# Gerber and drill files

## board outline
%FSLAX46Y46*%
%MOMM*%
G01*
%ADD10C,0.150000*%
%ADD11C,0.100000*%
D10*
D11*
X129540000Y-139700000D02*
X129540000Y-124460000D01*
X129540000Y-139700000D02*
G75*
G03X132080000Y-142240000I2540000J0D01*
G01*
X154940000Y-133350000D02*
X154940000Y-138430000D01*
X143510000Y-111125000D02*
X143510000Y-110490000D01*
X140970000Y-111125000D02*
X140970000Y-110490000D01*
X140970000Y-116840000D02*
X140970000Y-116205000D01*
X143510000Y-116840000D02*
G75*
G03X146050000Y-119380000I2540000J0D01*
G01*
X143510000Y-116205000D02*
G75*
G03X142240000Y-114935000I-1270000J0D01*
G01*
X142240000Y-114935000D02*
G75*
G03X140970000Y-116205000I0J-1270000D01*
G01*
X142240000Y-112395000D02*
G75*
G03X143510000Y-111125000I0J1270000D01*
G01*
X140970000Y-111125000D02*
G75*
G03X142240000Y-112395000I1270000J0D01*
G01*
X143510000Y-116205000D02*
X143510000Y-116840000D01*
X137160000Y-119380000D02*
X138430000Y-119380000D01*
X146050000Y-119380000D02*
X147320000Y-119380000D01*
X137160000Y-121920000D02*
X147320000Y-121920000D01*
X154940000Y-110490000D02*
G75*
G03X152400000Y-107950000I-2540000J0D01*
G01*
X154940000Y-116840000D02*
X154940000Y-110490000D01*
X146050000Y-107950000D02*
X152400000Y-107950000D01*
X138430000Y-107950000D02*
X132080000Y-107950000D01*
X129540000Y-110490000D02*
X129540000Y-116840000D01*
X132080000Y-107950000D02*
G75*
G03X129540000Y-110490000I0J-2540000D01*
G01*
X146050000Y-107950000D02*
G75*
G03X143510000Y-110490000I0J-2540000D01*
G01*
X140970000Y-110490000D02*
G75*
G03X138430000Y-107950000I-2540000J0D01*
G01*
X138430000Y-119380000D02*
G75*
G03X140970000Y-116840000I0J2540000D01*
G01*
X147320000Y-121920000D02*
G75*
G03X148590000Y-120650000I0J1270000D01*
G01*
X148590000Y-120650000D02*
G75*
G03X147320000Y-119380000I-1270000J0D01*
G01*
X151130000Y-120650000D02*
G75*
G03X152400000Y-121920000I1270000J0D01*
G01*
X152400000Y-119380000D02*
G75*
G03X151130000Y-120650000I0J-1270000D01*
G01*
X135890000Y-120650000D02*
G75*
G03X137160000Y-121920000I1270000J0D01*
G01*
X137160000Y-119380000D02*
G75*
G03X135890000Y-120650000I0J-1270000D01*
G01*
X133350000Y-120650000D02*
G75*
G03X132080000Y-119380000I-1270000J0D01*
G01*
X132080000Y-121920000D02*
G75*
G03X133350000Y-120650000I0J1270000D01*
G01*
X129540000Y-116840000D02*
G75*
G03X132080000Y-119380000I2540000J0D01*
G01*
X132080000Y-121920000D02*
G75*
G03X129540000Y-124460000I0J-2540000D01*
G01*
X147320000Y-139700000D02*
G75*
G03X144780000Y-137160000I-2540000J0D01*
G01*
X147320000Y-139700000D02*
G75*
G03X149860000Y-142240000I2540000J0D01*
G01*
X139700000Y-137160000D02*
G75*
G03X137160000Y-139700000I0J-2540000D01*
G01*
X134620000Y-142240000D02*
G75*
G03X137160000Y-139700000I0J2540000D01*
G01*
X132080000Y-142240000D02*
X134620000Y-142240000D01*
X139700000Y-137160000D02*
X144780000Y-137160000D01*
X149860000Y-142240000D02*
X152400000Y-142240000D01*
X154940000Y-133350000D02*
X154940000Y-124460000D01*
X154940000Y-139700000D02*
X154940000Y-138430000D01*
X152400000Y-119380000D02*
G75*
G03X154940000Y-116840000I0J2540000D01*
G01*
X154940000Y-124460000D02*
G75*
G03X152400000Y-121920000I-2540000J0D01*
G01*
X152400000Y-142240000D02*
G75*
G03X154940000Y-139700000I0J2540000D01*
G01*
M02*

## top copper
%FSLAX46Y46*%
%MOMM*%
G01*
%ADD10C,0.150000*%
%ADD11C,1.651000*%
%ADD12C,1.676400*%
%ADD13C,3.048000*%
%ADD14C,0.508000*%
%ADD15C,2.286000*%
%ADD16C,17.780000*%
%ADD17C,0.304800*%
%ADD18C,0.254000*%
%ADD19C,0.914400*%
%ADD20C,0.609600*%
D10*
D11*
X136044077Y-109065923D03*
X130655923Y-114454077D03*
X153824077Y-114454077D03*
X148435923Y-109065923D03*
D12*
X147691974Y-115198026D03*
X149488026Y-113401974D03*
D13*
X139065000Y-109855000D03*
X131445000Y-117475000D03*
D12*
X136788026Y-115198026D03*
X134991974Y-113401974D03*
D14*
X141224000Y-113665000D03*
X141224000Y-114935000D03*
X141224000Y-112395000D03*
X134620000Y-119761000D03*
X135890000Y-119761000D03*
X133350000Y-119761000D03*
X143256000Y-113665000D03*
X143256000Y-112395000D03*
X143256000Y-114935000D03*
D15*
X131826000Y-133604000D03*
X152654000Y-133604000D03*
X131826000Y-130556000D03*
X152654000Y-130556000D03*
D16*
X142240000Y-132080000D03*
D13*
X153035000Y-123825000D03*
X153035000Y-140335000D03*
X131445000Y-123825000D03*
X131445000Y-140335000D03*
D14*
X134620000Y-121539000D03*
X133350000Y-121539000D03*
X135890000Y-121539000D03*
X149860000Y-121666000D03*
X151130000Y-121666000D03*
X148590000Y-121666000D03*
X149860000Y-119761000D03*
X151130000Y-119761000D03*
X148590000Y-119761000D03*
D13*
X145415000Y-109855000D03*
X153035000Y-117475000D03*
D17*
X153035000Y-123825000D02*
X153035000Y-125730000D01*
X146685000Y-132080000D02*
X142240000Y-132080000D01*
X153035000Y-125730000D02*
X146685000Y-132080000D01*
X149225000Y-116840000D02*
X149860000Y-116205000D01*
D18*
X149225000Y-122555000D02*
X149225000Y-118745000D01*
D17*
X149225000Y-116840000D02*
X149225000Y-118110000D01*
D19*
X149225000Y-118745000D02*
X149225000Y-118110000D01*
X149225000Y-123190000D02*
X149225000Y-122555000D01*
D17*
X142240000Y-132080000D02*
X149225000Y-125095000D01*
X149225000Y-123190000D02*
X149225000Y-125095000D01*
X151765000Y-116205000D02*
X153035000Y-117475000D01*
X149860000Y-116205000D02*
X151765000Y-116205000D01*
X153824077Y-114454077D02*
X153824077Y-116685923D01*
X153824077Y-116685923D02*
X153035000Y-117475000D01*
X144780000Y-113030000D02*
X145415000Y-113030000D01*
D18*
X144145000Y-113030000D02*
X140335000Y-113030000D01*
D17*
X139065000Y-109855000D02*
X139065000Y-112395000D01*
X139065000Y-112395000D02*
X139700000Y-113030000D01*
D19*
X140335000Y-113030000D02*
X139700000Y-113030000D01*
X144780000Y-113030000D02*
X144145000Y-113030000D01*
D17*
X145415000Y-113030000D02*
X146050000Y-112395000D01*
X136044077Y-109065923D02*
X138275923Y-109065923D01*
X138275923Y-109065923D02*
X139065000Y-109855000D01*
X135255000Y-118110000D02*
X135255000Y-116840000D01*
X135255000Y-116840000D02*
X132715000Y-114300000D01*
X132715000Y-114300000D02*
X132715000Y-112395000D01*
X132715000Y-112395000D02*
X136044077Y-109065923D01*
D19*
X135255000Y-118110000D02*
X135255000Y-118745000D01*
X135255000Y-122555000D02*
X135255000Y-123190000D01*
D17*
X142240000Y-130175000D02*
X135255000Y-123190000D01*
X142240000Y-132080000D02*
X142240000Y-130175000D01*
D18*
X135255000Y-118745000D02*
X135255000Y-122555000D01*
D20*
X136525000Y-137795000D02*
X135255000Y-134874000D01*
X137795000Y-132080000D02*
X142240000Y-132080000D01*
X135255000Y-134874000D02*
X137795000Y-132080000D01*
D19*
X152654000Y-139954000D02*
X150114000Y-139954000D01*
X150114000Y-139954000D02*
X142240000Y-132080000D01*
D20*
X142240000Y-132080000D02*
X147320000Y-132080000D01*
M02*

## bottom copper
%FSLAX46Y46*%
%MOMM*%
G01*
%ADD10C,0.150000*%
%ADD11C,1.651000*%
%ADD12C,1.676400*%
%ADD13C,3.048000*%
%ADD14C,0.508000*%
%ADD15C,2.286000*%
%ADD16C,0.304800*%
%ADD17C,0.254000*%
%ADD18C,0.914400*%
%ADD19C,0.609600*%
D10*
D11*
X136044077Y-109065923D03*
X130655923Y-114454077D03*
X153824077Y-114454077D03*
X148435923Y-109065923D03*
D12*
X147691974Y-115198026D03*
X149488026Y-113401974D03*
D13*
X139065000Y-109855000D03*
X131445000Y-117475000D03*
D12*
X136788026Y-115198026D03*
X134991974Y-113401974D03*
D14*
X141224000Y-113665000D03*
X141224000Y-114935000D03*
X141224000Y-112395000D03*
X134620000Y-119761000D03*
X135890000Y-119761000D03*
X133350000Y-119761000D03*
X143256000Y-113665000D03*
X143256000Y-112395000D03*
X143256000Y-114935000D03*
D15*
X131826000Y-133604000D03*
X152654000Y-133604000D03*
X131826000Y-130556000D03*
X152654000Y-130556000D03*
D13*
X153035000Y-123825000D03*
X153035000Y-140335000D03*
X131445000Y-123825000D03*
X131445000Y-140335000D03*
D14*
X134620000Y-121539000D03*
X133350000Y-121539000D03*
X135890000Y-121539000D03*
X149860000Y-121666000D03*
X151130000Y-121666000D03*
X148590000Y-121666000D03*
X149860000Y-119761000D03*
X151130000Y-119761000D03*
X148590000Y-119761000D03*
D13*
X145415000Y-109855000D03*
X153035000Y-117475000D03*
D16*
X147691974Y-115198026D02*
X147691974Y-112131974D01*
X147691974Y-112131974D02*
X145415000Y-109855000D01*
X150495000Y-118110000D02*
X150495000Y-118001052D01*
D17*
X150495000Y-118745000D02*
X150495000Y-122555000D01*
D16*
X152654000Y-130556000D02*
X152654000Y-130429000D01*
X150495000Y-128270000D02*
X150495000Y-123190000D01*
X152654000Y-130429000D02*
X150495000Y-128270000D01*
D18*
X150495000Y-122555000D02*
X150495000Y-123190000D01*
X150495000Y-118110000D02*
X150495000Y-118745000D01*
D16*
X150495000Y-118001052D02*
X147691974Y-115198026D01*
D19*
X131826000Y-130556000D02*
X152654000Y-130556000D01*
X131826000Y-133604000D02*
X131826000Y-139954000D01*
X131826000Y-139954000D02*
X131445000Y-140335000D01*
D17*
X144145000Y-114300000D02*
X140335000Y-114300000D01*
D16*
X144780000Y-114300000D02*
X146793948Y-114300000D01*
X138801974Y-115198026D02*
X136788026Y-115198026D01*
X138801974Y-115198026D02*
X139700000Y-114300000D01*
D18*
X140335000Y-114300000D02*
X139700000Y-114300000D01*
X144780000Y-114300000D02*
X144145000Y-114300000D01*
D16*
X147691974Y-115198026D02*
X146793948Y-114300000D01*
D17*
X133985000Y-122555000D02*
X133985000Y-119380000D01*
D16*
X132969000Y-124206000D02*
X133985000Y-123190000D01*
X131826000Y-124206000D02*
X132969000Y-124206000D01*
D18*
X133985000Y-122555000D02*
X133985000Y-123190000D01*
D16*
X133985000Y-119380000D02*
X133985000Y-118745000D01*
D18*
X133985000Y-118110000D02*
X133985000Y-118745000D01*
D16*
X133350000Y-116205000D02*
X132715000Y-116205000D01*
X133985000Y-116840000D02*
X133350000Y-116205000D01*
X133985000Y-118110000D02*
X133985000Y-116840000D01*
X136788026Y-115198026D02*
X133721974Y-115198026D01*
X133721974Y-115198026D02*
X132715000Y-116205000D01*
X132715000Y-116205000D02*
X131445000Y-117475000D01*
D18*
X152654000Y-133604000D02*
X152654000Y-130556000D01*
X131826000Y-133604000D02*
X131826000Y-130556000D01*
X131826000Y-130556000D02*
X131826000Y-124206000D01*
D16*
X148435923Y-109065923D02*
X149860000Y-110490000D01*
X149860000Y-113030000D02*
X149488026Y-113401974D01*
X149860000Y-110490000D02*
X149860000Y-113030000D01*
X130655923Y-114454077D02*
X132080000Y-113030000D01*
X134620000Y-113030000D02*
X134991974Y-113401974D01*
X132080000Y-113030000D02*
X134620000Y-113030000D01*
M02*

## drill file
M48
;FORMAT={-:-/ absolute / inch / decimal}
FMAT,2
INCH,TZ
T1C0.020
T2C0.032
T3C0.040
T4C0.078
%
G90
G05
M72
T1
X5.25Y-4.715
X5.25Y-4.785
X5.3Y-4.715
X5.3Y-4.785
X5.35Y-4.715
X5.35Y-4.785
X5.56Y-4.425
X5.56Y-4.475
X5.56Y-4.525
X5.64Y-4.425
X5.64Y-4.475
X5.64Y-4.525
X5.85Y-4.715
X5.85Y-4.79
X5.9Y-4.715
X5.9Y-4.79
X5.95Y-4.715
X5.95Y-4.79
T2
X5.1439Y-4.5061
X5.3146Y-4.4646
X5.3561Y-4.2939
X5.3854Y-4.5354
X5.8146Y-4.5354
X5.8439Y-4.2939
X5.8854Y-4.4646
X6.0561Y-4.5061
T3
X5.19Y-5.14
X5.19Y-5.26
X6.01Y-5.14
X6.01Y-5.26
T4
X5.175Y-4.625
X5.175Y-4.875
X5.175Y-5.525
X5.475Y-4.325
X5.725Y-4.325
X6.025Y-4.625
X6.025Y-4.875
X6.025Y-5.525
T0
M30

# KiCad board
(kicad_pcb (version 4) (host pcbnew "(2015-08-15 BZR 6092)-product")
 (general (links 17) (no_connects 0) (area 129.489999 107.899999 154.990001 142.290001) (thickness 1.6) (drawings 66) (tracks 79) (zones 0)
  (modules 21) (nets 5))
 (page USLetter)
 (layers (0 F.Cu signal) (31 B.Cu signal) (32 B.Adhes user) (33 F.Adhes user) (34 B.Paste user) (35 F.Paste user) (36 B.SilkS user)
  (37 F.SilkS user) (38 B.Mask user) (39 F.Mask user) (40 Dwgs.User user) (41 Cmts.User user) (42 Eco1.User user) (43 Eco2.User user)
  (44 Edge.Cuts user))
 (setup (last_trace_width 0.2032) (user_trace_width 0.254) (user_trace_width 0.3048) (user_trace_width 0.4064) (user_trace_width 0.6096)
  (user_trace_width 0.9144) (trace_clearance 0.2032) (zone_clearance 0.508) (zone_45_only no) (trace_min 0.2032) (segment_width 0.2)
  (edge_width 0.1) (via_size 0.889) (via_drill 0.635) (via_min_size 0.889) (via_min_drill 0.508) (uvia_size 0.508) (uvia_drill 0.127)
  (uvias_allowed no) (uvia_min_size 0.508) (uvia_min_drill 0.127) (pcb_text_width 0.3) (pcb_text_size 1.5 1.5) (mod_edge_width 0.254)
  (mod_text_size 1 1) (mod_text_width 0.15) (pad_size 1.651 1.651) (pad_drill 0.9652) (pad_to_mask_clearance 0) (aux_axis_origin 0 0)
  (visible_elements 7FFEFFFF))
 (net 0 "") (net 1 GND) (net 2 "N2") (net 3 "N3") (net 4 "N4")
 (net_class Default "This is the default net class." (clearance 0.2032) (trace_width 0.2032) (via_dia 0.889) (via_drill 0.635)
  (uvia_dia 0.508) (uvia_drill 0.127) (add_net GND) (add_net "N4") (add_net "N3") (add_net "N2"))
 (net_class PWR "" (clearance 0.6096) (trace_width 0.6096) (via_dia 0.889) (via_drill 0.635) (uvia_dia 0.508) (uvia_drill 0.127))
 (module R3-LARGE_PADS (layer F.Cu) (at 133.35 111.76 225) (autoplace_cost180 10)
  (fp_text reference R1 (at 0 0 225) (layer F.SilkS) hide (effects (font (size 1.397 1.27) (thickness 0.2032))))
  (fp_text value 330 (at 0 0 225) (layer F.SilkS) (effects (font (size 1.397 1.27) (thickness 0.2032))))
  (pad 1 thru_hole circle (at -3.81 0 225) (size 1.651 1.651) (drill 0.8128) (layers *.Cu *.Mask F.SilkS) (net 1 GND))
  (pad 2 thru_hole circle (at 3.81 0 225) (size 1.651 1.651) (drill 0.8128) (layers *.Cu *.Mask F.SilkS) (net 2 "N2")))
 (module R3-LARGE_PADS (layer F.Cu) (at 151.13 111.76 135) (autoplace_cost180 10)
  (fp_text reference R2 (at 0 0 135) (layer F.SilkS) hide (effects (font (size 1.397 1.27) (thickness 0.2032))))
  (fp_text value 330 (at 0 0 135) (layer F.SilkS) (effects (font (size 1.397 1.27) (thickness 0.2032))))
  (pad 1 thru_hole circle (at -3.81 0 135) (size 1.651 1.651) (drill 0.8128) (layers *.Cu *.Mask F.SilkS) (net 1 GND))
  (pad 2 thru_hole circle (at 3.81 0 135) (size 1.651 1.651) (drill 0.8128) (layers *.Cu *.Mask F.SilkS) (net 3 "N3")))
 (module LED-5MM (layer F.Cu) (at 148.59 114.3 45)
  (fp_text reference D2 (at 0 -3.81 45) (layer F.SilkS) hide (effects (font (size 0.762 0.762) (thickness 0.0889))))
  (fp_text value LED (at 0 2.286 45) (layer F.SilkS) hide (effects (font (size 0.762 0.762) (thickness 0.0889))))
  (pad 1 thru_hole circle (at -1.27 0 45) (size 1.6764 1.6764) (drill 0.8128) (layers *.Cu *.Mask F.SilkS) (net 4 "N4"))
  (pad 2 thru_hole circle (at 1.27 0 45) (size 1.6764 1.6764) (drill 0.8128) (layers *.Cu *.Mask F.SilkS) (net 3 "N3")))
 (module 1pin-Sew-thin (layer F.Cu) (at 139.065 109.855 270)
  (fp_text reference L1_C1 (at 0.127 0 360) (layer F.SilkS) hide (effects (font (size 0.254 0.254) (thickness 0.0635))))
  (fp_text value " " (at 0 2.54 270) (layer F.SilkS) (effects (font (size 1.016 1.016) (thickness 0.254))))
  (pad 1 thru_hole circle (at 0 0 270) (size 3.048 3.048) (drill 1.984375) (layers *.Cu *.Mask F.SilkS) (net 1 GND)))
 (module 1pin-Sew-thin (layer F.Cu) (at 131.445 117.475 270)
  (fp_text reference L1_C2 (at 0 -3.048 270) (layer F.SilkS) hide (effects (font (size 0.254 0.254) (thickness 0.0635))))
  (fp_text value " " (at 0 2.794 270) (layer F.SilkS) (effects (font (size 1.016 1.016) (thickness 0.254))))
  (pad 1 thru_hole circle (at 0 0 270) (size 3.048 3.048) (drill 1.984375) (layers *.Cu *.Mask F.SilkS) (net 4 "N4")))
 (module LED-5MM (layer F.Cu) (at 135.89 114.3 135)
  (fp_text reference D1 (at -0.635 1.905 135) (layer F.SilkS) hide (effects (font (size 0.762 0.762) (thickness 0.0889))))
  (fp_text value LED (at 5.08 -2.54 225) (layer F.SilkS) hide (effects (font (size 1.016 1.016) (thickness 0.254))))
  (pad 1 thru_hole circle (at -1.27 0 135) (size 1.6764 1.6764) (drill 0.8128) (layers *.Cu *.Mask F.SilkS) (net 4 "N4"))
  (pad 2 thru_hole circle (at 1.27 0 135) (size 1.6764 1.6764) (drill 0.8128) (layers *.Cu *.Mask F.SilkS) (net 2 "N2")))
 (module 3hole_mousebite (layer F.Cu) (at 141.605 113.665 90)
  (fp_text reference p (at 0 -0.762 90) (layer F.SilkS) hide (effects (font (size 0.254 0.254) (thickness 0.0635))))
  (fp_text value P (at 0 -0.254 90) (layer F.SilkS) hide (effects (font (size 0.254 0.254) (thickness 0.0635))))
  (pad "" thru_hole circle (at 0 -0.381 90) (size 0.508 0.508) (drill 0.508) (layers *.Cu *.Mask F.SilkS))
  (pad 1 thru_hole circle (at -1.27 -0.381 90) (size 0.508 0.508) (drill 0.508) (layers *.Cu *.Mask F.SilkS))
  (pad 2 thru_hole circle (at 1.27 -0.381 90) (size 0.508 0.508) (drill 0.508) (layers *.Cu *.Mask F.SilkS)))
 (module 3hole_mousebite (layer F.Cu) (at 134.62 119.38 180)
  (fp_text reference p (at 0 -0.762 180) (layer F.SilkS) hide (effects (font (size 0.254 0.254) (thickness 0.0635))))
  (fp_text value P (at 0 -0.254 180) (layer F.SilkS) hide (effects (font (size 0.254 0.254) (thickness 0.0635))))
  (pad "" thru_hole circle (at 0 -0.381 180) (size 0.508 0.508) (drill 0.508) (layers *.Cu *.Mask F.SilkS))
  (pad 1 thru_hole circle (at -1.27 -0.381 180) (size 0.508 0.508) (drill 0.508) (layers *.Cu *.Mask F.SilkS))
  (pad 2 thru_hole circle (at 1.27 -0.381 180) (size 0.508 0.508) (drill 0.508) (layers *.Cu *.Mask F.SilkS)))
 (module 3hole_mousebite (layer F.Cu) (at 142.875 113.665 270)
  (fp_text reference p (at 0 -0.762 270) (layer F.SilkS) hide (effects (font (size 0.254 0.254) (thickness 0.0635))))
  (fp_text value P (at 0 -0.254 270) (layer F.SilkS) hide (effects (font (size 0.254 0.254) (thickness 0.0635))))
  (pad "" thru_hole circle (at 0 -0.381 270) (size 0.508 0.508) (drill 0.508) (layers *.Cu *.Mask F.SilkS))
  (pad 1 thru_hole circle (at -1.27 -0.381 270) (size 0.508 0.508) (drill 0.508) (layers *.Cu *.Mask F.SilkS))
  (pad 2 thru_hole circle (at 1.27 -0.381 270) (size 0.508 0.508) (drill 0.508) (layers *.Cu *.Mask F.SilkS)))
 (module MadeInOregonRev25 (layer F.Cu) (at 137.033 131.699)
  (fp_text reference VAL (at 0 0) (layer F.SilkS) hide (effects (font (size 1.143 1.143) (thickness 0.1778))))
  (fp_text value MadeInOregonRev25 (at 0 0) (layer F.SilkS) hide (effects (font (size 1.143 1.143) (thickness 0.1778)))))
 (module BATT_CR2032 (layer F.Cu) (at 142.24 132.08)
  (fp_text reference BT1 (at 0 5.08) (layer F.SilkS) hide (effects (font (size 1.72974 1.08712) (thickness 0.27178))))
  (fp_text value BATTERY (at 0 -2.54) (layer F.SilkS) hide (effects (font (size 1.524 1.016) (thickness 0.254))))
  (pad 1 thru_hole circle (at -10.414 1.524) (size 2.286 2.286) (drill 1.016) (layers *.Cu *.Mask F.SilkS) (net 4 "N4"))
  (pad 1 thru_hole circle (at 10.414 1.524) (size 2.286 2.286) (drill 1.016) (layers *.Cu *.Mask F.SilkS) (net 4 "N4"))
  (pad 1 thru_hole circle (at -10.414 -1.524) (size 2.286 2.286) (drill 1.016) (layers *.Cu *.Mask F.SilkS) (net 4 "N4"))
  (pad 1 thru_hole circle (at 10.414 -1.524) (size 2.286 2.286) (drill 1.016) (layers *.Cu *.Mask F.SilkS) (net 4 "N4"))
  (pad 2 smd circle (at 0 0) (size 17.78 17.78) (layers F.Cu F.Paste F.Mask) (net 1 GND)))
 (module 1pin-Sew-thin (layer F.Cu) (at 153.035 123.825)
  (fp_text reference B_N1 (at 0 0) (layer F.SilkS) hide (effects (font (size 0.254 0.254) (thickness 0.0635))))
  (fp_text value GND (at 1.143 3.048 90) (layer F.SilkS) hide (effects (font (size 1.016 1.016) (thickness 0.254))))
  (pad 1 thru_hole circle (at 0 0) (size 3.048 3.048) (drill 1.984375) (layers *.Cu *.Mask F.SilkS) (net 1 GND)))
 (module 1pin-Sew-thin (layer F.Cu) (at 153.035 140.335)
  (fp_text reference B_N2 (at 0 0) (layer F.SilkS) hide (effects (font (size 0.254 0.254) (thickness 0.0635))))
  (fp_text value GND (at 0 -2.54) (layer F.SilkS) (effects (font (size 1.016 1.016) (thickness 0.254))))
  (pad 1 thru_hole circle (at 0 0) (size 3.048 3.048) (drill 1.984375) (layers *.Cu *.Mask F.SilkS) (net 1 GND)))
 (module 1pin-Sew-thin (layer F.Cu) (at 131.445 123.825)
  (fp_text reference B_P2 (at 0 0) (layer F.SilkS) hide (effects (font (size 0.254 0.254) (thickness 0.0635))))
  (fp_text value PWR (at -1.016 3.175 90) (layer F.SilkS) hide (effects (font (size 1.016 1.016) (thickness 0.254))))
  (pad 1 thru_hole circle (at 0 0) (size 3.048 3.048) (drill 1.984375) (layers *.Cu *.Mask F.SilkS) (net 4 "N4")))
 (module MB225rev (layer F.Cu) (at 147.447 131.699)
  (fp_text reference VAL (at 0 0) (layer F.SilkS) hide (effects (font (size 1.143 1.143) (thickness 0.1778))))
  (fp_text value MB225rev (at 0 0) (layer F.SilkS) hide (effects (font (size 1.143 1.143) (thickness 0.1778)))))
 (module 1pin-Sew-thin (layer F.Cu) (at 131.445 140.335)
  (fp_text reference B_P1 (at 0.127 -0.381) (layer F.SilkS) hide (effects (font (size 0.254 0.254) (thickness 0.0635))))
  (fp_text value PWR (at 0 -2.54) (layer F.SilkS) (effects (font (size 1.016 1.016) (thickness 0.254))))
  (pad 1 thru_hole circle (at 0 0) (size 3.048 3.048) (drill 1.984375) (layers *.Cu *.Mask F.SilkS) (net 4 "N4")))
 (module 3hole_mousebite (layer F.Cu) (at 134.62 121.92)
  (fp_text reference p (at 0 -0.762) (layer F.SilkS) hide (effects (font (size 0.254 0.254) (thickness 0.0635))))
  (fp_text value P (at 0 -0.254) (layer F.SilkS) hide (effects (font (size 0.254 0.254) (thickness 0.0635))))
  (pad "" thru_hole circle (at 0 -0.381) (size 0.508 0.508) (drill 0.508) (layers *.Cu *.Mask F.SilkS))
  (pad 1 thru_hole circle (at -1.27 -0.381) (size 0.508 0.508) (drill 0.508) (layers *.Cu *.Mask F.SilkS))
  (pad 2 thru_hole circle (at 1.27 -0.381) (size 0.508 0.508) (drill 0.508) (layers *.Cu *.Mask F.SilkS)))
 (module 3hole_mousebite (layer F.Cu) (at 149.86 121.285 180)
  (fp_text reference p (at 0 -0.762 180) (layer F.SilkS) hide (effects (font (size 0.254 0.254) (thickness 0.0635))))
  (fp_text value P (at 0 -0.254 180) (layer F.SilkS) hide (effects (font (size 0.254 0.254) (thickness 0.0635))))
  (pad "" thru_hole circle (at 0 -0.381 180) (size 0.508 0.508) (drill 0.508) (layers *.Cu *.Mask F.SilkS))
  (pad 1 thru_hole circle (at -1.27 -0.381 180) (size 0.508 0.508) (drill 0.508) (layers *.Cu *.Mask F.SilkS))
  (pad 2 thru_hole circle (at 1.27 -0.381 180) (size 0.508 0.508) (drill 0.508) (layers *.Cu *.Mask F.SilkS)))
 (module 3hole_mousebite (layer F.Cu) (at 149.86 119.38 180)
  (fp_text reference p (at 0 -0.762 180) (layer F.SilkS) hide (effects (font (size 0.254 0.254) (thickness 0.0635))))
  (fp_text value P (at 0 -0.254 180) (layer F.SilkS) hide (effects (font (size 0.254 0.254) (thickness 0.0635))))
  (pad "" thru_hole circle (at 0 -0.381 180) (size 0.508 0.508) (drill 0.508) (layers *.Cu *.Mask F.SilkS))
  (pad 1 thru_hole circle (at -1.27 -0.381 180) (size 0.508 0.508) (drill 0.508) (layers *.Cu *.Mask F.SilkS))
  (pad 2 thru_hole circle (at 1.27 -0.381 180) (size 0.508 0.508) (drill 0.508) (layers *.Cu *.Mask F.SilkS)))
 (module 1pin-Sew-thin (layer F.Cu) (at 145.415 109.855)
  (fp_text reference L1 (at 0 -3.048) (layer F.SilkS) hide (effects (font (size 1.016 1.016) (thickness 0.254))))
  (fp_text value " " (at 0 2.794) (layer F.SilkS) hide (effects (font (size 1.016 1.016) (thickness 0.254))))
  (pad 1 thru_hole circle (at 0 0) (size 3.048 3.048) (drill 1.984375) (layers *.Cu *.Mask F.SilkS) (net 4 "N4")))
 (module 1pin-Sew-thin (layer F.Cu) (at 153.035 117.475)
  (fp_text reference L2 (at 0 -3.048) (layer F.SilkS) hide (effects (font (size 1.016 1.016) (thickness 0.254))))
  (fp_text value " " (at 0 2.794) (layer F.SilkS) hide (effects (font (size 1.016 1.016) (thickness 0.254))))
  (pad 1 thru_hole circle (at 0 0) (size 3.048 3.048) (drill 1.984375) (layers *.Cu *.Mask F.SilkS) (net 1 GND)))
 (gr_line (start 129.54 139.7) (end 129.54 124.46) (angle 90) (layer Edge.Cuts) (width 0.1))
 (gr_arc (start 132.08 139.7) (end 132.08 142.24) (angle 90) (layer Edge.Cuts) (width 0.1))
 (gr_line (start 154.94 133.35) (end 154.94 138.43) (angle 90) (layer Edge.Cuts) (width 0.1))
 (gr_line (start 143.51 111.125) (end 143.51 110.49) (angle 90) (layer Edge.Cuts) (width 0.1))
 (gr_line (start 140.97 111.125) (end 140.97 110.49) (angle 90) (layer Edge.Cuts) (width 0.1))
 (gr_line (start 140.97 116.84) (end 140.97 116.205) (angle 90) (layer Edge.Cuts) (width 0.1))
 (gr_arc (start 146.05 116.84) (end 146.05 119.38) (angle 90) (layer Edge.Cuts) (width 0.1))
 (gr_arc (start 142.24 116.205) (end 142.24 114.935) (angle 90) (layer Edge.Cuts) (width 0.1))
 (gr_arc (start 142.24 116.205) (end 140.97 116.205) (angle 90) (layer Edge.Cuts) (width 0.1))
 (gr_arc (start 142.24 111.125) (end 143.51 111.125) (angle 90) (layer Edge.Cuts) (width 0.1))
 (gr_arc (start 142.24 111.125) (end 142.24 112.395) (angle 90) (layer Edge.Cuts) (width 0.1))
 (gr_line (start 143.51 116.205) (end 143.51 116.84) (angle 90) (layer Edge.Cuts) (width 0.1))
 (gr_line (start 137.16 119.38) (end 138.43 119.38) (angle 90) (layer Edge.Cuts) (width 0.1))
 (gr_line (start 146.05 119.38) (end 147.32 119.38) (angle 90) (layer Edge.Cuts) (width 0.1))
 (gr_line (start 137.16 121.92) (end 147.32 121.92) (angle 90) (layer Edge.Cuts) (width 0.1))
 (gr_arc (start 152.4 110.49) (end 152.4 107.95) (angle 90) (layer Edge.Cuts) (width 0.1))
 (gr_line (start 154.94 116.84) (end 154.94 110.49) (angle 90) (layer Edge.Cuts) (width 0.1))
 (gr_line (start 146.05 107.95) (end 152.4 107.95) (angle 90) (layer Edge.Cuts) (width 0.1))
 (gr_line (start 138.43 107.95) (end 132.08 107.95) (angle 90) (layer Edge.Cuts) (width 0.1))
 (gr_line (start 129.54 110.49) (end 129.54 116.84) (angle 90) (layer Edge.Cuts) (width 0.1))
 (gr_arc (start 132.08 110.49) (end 129.54 110.49) (angle 90) (layer Edge.Cuts) (width 0.1))
 (gr_arc (start 146.05 110.49) (end 143.51 110.49) (angle 90) (layer Edge.Cuts) (width 0.1))
 (gr_arc (start 138.43 110.49) (end 138.43 107.95) (angle 90) (layer Edge.Cuts) (width 0.1))
 (gr_arc (start 138.43 116.84) (end 140.97 116.84) (angle 90) (layer Edge.Cuts) (width 0.1))
 (gr_arc (start 147.32 120.65) (end 148.59 120.65) (angle 90) (layer Edge.Cuts) (width 0.1))
 (gr_arc (start 147.32 120.65) (end 147.32 119.38) (angle 90) (layer Edge.Cuts) (width 0.1))
 (gr_arc (start 152.4 120.65) (end 152.4 121.92) (angle 90) (layer Edge.Cuts) (width 0.1))
 (gr_arc (start 152.4 120.65) (end 151.13 120.65) (angle 90) (layer Edge.Cuts) (width 0.1))
 (gr_arc (start 137.16 120.65) (end 137.16 121.92) (angle 90) (layer Edge.Cuts) (width 0.1))
 (gr_arc (start 137.16 120.65) (end 135.89 120.65) (angle 90) (layer Edge.Cuts) (width 0.1))
 (gr_arc (start 132.08 120.65) (end 132.08 119.38) (angle 90) (layer Edge.Cuts) (width 0.1))
 (gr_arc (start 132.08 120.65) (end 133.35 120.65) (angle 90) (layer Edge.Cuts) (width 0.1))
 (gr_arc (start 132.08 116.84) (end 132.08 119.38) (angle 90) (layer Edge.Cuts) (width 0.1))
 (gr_arc (start 132.08 124.46) (end 129.54 124.46) (angle 90) (layer Edge.Cuts) (width 0.1))
 (gr_arc (start 144.78 139.7) (end 144.78 137.16) (angle 90) (layer Edge.Cuts) (width 0.1))
 (gr_arc (start 149.86 139.7) (end 149.86 142.24) (angle 90) (layer Edge.Cuts) (width 0.1))
 (gr_arc (start 139.7 139.7) (end 137.16 139.7) (angle 90) (layer Edge.Cuts) (width 0.1))
 (gr_arc (start 134.62 139.7) (end 137.16 139.7) (angle 90) (layer Edge.Cuts) (width 0.1))
 (gr_line (start 132.08 142.24) (end 134.62 142.24) (angle 90) (layer Edge.Cuts) (width 0.1))
 (gr_line (start 139.7 137.16) (end 144.78 137.16) (angle 90) (layer Edge.Cuts) (width 0.1))
 (gr_line (start 149.86 142.24) (end 152.4 142.24) (angle 90) (layer Edge.Cuts) (width 0.1))
 (gr_line (start 154.94 133.35) (end 154.94 124.46) (angle 90) (layer Edge.Cuts) (width 0.1))
 (gr_line (start 154.94 139.7) (end 154.94 138.43) (angle 90) (layer Edge.Cuts) (width 0.1))
 (gr_arc (start 152.4 116.84) (end 154.94 116.84) (angle 90) (layer Edge.Cuts) (width 0.1))
 (gr_arc (start 152.4 124.46) (end 152.4 121.92) (angle 90) (layer Edge.Cuts) (width 0.1))
 (gr_arc (start 152.4 139.7) (end 154.94 139.7) (angle 90) (layer Edge.Cuts) (width 0.1))
 (segment (start 153.035 123.825) (end 153.035 125.73) (width 0.3048) (layer F.Cu) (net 1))
 (segment (start 146.685 132.08) (end 142.24 132.08) (width 0.3048) (layer F.Cu) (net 1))
 (segment (start 153.035 125.73) (end 146.685 132.08) (width 0.3048) (layer F.Cu) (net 1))
 (segment (start 149.225 116.84) (end 149.86 116.205) (width 0.3048) (layer F.Cu) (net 1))
 (segment (start 149.225 122.555) (end 149.225 118.745) (width 0.254) (layer F.Cu) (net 1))
 (segment (start 149.225 116.84) (end 149.225 118.11) (width 0.3048) (layer F.Cu) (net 1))
 (segment (start 149.225 118.745) (end 149.225 118.11) (width 0.9144) (layer F.Cu) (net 1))
 (segment (start 149.225 123.19) (end 149.225 122.555) (width 0.9144) (layer F.Cu) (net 1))
 (segment (start 142.24 132.08) (end 149.225 125.095) (width 0.3048) (layer F.Cu) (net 1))
 (segment (start 149.225 123.19) (end 149.225 125.095) (width 0.3048) (layer F.Cu) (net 1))
 (segment (start 151.765 116.205) (end 153.035 117.475) (width 0.3048) (layer F.Cu) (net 1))
 (segment (start 149.86 116.205) (end 151.765 116.205) (width 0.3048) (layer F.Cu) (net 1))
 (segment (start 153.824077 114.454077) (end 153.824077 116.685923) (width 0.3048) (layer F.Cu) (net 1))
 (segment (start 153.824077 116.685923) (end 153.035 117.475) (width 0.3048) (layer F.Cu) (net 1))
 (segment (start 144.78 113.03) (end 145.415 113.03) (width 0.3048) (layer F.Cu) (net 1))
 (segment (start 144.145 113.03) (end 140.335 113.03) (width 0.254) (layer F.Cu) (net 1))
 (segment (start 139.065 109.855) (end 139.065 112.395) (width 0.3048) (layer F.Cu) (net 1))
 (segment (start 139.065 112.395) (end 139.7 113.03) (width 0.3048) (layer F.Cu) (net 1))
 (segment (start 140.335 113.03) (end 139.7 113.03) (width 0.9144) (layer F.Cu) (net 1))
 (segment (start 144.78 113.03) (end 144.145 113.03) (width 0.9144) (layer F.Cu) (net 1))
 (segment (start 145.415 113.03) (end 146.05 112.395) (width 0.3048) (layer F.Cu) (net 1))
 (segment (start 136.044077 109.065923) (end 138.275923 109.065923) (width 0.3048) (layer F.Cu) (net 1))
 (segment (start 138.275923 109.065923) (end 139.065 109.855) (width 0.3048) (layer F.Cu) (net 1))
 (segment (start 135.255 118.11) (end 135.255 116.84) (width 0.3048) (layer F.Cu) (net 1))
 (segment (start 135.255 116.84) (end 132.715 114.3) (width 0.3048) (layer F.Cu) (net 1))
 (segment (start 132.715 114.3) (end 132.715 112.395) (width 0.3048) (layer F.Cu) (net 1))
 (segment (start 132.715 112.395) (end 136.044077 109.065923) (width 0.3048) (layer F.Cu) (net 1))
 (segment (start 135.255 118.11) (end 135.255 118.745) (width 0.9144) (layer F.Cu) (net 1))
 (segment (start 135.255 122.555) (end 135.255 123.19) (width 0.9144) (layer F.Cu) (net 1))
 (segment (start 142.24 130.175) (end 135.255 123.19) (width 0.3048) (layer F.Cu) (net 1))
 (segment (start 142.24 132.08) (end 142.24 130.175) (width 0.3048) (layer F.Cu) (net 1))
 (segment (start 135.255 118.745) (end 135.255 122.555) (width 0.254) (layer F.Cu) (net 1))
 (segment (start 136.525 137.795) (end 135.255 134.874) (width 0.6096) (layer F.Cu) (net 1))
 (segment (start 137.795 132.08) (end 142.24 132.08) (width 0.6096) (layer F.Cu) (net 1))
 (segment (start 135.255 134.874) (end 137.795 132.08) (width 0.6096) (layer F.Cu) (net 1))
 (segment (start 152.654 139.954) (end 150.114 139.954) (width 0.9144) (layer F.Cu) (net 1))
 (segment (start 150.114 139.954) (end 142.24 132.08) (width 0.9144) (layer F.Cu) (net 1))
 (segment (start 142.24 132.08) (end 147.32 132.08) (width 0.6096) (layer F.Cu) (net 1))
 (segment (start 147.691974 115.198026) (end 147.691974 112.131974) (width 0.3048) (layer B.Cu) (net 4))
 (segment (start 147.691974 112.131974) (end 145.415 109.855) (width 0.3048) (layer B.Cu) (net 4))
 (segment (start 150.495 118.11) (end 150.495 118.001052) (width 0.3048) (layer B.Cu) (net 4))
 (segment (start 150.495 118.745) (end 150.495 122.555) (width 0.254) (layer B.Cu) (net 4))
 (segment (start 152.654 130.556) (end 152.654 130.429) (width 0.3048) (layer B.Cu) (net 4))
 (segment (start 150.495 128.27) (end 150.495 123.19) (width 0.3048) (layer B.Cu) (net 4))
 (segment (start 152.654 130.429) (end 150.495 128.27) (width 0.3048) (layer B.Cu) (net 4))
 (segment (start 150.495 122.555) (end 150.495 123.19) (width 0.9144) (layer B.Cu) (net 4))
 (segment (start 150.495 118.11) (end 150.495 118.745) (width 0.9144) (layer B.Cu) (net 4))
 (segment (start 150.495 118.001052) (end 147.691974 115.198026) (width 0.3048) (layer B.Cu) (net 4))
 (segment (start 131.826 130.556) (end 152.654 130.556) (width 0.6096) (layer B.Cu) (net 4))
 (segment (start 131.826 133.604) (end 131.826 139.954) (width 0.6096) (layer B.Cu) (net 4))
 (segment (start 131.826 139.954) (end 131.445 140.335) (width 0.6096) (layer B.Cu) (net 4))
 (segment (start 144.145 114.3) (end 140.335 114.3) (width 0.254) (layer B.Cu) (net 4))
 (segment (start 144.78 114.3) (end 146.793948 114.3) (width 0.3048) (layer B.Cu) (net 4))
 (segment (start 138.801974 115.198026) (end 136.788026 115.198026) (width 0.3048) (layer B.Cu) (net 4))
 (segment (start 138.801974 115.198026) (end 139.7 114.3) (width 0.3048) (layer B.Cu) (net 4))
 (segment (start 140.335 114.3) (end 139.7 114.3) (width 0.9144) (layer B.Cu) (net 4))
 (segment (start 144.78 114.3) (end 144.145 114.3) (width 0.9144) (layer B.Cu) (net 4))
 (segment (start 147.691974 115.198026) (end 146.793948 114.3) (width 0.3048) (layer B.Cu) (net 4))
 (segment (start 133.985 122.555) (end 133.985 119.38) (width 0.254) (layer B.Cu) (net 4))
 (segment (start 132.969 124.206) (end 133.985 123.19) (width 0.3048) (layer B.Cu) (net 4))
 (segment (start 131.826 124.206) (end 132.969 124.206) (width 0.3048) (layer B.Cu) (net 4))
 (segment (start 133.985 122.555) (end 133.985 123.19) (width 0.9144) (layer B.Cu) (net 4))
 (segment (start 133.985 119.38) (end 133.985 118.745) (width 0.3048) (layer B.Cu) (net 4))
 (segment (start 133.985 118.11) (end 133.985 118.745) (width 0.9144) (layer B.Cu) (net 4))
 (segment (start 133.35 116.205) (end 132.715 116.205) (width 0.3048) (layer B.Cu) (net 4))
 (segment (start 133.985 116.84) (end 133.35 116.205) (width 0.3048) (layer B.Cu) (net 4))
 (segment (start 133.985 118.11) (end 133.985 116.84) (width 0.3048) (layer B.Cu) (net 4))
 (segment (start 136.788026 115.198026) (end 133.721974 115.198026) (width 0.3048) (layer B.Cu) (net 4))
 (segment (start 133.721974 115.198026) (end 132.715 116.205) (width 0.3048) (layer B.Cu) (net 4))
 (segment (start 132.715 116.205) (end 131.445 117.475) (width 0.3048) (layer B.Cu) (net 4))
 (segment (start 152.654 133.604) (end 152.654 130.556) (width 0.9144) (layer B.Cu) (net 4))
 (segment (start 131.826 133.604) (end 131.826 130.556) (width 0.9144) (layer B.Cu) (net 4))
 (segment (start 131.826 130.556) (end 131.826 124.206) (width 0.9144) (layer B.Cu) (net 4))
 (segment (start 148.435923 109.065923) (end 149.86 110.49) (width 0.3048) (layer B.Cu) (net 3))
 (segment (start 149.86 113.03) (end 149.488026 113.401974) (width 0.3048) (layer B.Cu) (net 3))
 (segment (start 149.86 110.49) (end 149.86 113.03) (width 0.3048) (layer B.Cu) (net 3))
 (segment (start 130.655923 114.454077) (end 132.08 113.03) (width 0.3048) (layer B.Cu) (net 2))
 (segment (start 134.62 113.03) (end 134.991974 113.401974) (width 0.3048) (layer B.Cu) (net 2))
 (segment (start 132.08 113.03) (end 134.62 113.03) (width 0.3048) (layer B.Cu) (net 2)))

